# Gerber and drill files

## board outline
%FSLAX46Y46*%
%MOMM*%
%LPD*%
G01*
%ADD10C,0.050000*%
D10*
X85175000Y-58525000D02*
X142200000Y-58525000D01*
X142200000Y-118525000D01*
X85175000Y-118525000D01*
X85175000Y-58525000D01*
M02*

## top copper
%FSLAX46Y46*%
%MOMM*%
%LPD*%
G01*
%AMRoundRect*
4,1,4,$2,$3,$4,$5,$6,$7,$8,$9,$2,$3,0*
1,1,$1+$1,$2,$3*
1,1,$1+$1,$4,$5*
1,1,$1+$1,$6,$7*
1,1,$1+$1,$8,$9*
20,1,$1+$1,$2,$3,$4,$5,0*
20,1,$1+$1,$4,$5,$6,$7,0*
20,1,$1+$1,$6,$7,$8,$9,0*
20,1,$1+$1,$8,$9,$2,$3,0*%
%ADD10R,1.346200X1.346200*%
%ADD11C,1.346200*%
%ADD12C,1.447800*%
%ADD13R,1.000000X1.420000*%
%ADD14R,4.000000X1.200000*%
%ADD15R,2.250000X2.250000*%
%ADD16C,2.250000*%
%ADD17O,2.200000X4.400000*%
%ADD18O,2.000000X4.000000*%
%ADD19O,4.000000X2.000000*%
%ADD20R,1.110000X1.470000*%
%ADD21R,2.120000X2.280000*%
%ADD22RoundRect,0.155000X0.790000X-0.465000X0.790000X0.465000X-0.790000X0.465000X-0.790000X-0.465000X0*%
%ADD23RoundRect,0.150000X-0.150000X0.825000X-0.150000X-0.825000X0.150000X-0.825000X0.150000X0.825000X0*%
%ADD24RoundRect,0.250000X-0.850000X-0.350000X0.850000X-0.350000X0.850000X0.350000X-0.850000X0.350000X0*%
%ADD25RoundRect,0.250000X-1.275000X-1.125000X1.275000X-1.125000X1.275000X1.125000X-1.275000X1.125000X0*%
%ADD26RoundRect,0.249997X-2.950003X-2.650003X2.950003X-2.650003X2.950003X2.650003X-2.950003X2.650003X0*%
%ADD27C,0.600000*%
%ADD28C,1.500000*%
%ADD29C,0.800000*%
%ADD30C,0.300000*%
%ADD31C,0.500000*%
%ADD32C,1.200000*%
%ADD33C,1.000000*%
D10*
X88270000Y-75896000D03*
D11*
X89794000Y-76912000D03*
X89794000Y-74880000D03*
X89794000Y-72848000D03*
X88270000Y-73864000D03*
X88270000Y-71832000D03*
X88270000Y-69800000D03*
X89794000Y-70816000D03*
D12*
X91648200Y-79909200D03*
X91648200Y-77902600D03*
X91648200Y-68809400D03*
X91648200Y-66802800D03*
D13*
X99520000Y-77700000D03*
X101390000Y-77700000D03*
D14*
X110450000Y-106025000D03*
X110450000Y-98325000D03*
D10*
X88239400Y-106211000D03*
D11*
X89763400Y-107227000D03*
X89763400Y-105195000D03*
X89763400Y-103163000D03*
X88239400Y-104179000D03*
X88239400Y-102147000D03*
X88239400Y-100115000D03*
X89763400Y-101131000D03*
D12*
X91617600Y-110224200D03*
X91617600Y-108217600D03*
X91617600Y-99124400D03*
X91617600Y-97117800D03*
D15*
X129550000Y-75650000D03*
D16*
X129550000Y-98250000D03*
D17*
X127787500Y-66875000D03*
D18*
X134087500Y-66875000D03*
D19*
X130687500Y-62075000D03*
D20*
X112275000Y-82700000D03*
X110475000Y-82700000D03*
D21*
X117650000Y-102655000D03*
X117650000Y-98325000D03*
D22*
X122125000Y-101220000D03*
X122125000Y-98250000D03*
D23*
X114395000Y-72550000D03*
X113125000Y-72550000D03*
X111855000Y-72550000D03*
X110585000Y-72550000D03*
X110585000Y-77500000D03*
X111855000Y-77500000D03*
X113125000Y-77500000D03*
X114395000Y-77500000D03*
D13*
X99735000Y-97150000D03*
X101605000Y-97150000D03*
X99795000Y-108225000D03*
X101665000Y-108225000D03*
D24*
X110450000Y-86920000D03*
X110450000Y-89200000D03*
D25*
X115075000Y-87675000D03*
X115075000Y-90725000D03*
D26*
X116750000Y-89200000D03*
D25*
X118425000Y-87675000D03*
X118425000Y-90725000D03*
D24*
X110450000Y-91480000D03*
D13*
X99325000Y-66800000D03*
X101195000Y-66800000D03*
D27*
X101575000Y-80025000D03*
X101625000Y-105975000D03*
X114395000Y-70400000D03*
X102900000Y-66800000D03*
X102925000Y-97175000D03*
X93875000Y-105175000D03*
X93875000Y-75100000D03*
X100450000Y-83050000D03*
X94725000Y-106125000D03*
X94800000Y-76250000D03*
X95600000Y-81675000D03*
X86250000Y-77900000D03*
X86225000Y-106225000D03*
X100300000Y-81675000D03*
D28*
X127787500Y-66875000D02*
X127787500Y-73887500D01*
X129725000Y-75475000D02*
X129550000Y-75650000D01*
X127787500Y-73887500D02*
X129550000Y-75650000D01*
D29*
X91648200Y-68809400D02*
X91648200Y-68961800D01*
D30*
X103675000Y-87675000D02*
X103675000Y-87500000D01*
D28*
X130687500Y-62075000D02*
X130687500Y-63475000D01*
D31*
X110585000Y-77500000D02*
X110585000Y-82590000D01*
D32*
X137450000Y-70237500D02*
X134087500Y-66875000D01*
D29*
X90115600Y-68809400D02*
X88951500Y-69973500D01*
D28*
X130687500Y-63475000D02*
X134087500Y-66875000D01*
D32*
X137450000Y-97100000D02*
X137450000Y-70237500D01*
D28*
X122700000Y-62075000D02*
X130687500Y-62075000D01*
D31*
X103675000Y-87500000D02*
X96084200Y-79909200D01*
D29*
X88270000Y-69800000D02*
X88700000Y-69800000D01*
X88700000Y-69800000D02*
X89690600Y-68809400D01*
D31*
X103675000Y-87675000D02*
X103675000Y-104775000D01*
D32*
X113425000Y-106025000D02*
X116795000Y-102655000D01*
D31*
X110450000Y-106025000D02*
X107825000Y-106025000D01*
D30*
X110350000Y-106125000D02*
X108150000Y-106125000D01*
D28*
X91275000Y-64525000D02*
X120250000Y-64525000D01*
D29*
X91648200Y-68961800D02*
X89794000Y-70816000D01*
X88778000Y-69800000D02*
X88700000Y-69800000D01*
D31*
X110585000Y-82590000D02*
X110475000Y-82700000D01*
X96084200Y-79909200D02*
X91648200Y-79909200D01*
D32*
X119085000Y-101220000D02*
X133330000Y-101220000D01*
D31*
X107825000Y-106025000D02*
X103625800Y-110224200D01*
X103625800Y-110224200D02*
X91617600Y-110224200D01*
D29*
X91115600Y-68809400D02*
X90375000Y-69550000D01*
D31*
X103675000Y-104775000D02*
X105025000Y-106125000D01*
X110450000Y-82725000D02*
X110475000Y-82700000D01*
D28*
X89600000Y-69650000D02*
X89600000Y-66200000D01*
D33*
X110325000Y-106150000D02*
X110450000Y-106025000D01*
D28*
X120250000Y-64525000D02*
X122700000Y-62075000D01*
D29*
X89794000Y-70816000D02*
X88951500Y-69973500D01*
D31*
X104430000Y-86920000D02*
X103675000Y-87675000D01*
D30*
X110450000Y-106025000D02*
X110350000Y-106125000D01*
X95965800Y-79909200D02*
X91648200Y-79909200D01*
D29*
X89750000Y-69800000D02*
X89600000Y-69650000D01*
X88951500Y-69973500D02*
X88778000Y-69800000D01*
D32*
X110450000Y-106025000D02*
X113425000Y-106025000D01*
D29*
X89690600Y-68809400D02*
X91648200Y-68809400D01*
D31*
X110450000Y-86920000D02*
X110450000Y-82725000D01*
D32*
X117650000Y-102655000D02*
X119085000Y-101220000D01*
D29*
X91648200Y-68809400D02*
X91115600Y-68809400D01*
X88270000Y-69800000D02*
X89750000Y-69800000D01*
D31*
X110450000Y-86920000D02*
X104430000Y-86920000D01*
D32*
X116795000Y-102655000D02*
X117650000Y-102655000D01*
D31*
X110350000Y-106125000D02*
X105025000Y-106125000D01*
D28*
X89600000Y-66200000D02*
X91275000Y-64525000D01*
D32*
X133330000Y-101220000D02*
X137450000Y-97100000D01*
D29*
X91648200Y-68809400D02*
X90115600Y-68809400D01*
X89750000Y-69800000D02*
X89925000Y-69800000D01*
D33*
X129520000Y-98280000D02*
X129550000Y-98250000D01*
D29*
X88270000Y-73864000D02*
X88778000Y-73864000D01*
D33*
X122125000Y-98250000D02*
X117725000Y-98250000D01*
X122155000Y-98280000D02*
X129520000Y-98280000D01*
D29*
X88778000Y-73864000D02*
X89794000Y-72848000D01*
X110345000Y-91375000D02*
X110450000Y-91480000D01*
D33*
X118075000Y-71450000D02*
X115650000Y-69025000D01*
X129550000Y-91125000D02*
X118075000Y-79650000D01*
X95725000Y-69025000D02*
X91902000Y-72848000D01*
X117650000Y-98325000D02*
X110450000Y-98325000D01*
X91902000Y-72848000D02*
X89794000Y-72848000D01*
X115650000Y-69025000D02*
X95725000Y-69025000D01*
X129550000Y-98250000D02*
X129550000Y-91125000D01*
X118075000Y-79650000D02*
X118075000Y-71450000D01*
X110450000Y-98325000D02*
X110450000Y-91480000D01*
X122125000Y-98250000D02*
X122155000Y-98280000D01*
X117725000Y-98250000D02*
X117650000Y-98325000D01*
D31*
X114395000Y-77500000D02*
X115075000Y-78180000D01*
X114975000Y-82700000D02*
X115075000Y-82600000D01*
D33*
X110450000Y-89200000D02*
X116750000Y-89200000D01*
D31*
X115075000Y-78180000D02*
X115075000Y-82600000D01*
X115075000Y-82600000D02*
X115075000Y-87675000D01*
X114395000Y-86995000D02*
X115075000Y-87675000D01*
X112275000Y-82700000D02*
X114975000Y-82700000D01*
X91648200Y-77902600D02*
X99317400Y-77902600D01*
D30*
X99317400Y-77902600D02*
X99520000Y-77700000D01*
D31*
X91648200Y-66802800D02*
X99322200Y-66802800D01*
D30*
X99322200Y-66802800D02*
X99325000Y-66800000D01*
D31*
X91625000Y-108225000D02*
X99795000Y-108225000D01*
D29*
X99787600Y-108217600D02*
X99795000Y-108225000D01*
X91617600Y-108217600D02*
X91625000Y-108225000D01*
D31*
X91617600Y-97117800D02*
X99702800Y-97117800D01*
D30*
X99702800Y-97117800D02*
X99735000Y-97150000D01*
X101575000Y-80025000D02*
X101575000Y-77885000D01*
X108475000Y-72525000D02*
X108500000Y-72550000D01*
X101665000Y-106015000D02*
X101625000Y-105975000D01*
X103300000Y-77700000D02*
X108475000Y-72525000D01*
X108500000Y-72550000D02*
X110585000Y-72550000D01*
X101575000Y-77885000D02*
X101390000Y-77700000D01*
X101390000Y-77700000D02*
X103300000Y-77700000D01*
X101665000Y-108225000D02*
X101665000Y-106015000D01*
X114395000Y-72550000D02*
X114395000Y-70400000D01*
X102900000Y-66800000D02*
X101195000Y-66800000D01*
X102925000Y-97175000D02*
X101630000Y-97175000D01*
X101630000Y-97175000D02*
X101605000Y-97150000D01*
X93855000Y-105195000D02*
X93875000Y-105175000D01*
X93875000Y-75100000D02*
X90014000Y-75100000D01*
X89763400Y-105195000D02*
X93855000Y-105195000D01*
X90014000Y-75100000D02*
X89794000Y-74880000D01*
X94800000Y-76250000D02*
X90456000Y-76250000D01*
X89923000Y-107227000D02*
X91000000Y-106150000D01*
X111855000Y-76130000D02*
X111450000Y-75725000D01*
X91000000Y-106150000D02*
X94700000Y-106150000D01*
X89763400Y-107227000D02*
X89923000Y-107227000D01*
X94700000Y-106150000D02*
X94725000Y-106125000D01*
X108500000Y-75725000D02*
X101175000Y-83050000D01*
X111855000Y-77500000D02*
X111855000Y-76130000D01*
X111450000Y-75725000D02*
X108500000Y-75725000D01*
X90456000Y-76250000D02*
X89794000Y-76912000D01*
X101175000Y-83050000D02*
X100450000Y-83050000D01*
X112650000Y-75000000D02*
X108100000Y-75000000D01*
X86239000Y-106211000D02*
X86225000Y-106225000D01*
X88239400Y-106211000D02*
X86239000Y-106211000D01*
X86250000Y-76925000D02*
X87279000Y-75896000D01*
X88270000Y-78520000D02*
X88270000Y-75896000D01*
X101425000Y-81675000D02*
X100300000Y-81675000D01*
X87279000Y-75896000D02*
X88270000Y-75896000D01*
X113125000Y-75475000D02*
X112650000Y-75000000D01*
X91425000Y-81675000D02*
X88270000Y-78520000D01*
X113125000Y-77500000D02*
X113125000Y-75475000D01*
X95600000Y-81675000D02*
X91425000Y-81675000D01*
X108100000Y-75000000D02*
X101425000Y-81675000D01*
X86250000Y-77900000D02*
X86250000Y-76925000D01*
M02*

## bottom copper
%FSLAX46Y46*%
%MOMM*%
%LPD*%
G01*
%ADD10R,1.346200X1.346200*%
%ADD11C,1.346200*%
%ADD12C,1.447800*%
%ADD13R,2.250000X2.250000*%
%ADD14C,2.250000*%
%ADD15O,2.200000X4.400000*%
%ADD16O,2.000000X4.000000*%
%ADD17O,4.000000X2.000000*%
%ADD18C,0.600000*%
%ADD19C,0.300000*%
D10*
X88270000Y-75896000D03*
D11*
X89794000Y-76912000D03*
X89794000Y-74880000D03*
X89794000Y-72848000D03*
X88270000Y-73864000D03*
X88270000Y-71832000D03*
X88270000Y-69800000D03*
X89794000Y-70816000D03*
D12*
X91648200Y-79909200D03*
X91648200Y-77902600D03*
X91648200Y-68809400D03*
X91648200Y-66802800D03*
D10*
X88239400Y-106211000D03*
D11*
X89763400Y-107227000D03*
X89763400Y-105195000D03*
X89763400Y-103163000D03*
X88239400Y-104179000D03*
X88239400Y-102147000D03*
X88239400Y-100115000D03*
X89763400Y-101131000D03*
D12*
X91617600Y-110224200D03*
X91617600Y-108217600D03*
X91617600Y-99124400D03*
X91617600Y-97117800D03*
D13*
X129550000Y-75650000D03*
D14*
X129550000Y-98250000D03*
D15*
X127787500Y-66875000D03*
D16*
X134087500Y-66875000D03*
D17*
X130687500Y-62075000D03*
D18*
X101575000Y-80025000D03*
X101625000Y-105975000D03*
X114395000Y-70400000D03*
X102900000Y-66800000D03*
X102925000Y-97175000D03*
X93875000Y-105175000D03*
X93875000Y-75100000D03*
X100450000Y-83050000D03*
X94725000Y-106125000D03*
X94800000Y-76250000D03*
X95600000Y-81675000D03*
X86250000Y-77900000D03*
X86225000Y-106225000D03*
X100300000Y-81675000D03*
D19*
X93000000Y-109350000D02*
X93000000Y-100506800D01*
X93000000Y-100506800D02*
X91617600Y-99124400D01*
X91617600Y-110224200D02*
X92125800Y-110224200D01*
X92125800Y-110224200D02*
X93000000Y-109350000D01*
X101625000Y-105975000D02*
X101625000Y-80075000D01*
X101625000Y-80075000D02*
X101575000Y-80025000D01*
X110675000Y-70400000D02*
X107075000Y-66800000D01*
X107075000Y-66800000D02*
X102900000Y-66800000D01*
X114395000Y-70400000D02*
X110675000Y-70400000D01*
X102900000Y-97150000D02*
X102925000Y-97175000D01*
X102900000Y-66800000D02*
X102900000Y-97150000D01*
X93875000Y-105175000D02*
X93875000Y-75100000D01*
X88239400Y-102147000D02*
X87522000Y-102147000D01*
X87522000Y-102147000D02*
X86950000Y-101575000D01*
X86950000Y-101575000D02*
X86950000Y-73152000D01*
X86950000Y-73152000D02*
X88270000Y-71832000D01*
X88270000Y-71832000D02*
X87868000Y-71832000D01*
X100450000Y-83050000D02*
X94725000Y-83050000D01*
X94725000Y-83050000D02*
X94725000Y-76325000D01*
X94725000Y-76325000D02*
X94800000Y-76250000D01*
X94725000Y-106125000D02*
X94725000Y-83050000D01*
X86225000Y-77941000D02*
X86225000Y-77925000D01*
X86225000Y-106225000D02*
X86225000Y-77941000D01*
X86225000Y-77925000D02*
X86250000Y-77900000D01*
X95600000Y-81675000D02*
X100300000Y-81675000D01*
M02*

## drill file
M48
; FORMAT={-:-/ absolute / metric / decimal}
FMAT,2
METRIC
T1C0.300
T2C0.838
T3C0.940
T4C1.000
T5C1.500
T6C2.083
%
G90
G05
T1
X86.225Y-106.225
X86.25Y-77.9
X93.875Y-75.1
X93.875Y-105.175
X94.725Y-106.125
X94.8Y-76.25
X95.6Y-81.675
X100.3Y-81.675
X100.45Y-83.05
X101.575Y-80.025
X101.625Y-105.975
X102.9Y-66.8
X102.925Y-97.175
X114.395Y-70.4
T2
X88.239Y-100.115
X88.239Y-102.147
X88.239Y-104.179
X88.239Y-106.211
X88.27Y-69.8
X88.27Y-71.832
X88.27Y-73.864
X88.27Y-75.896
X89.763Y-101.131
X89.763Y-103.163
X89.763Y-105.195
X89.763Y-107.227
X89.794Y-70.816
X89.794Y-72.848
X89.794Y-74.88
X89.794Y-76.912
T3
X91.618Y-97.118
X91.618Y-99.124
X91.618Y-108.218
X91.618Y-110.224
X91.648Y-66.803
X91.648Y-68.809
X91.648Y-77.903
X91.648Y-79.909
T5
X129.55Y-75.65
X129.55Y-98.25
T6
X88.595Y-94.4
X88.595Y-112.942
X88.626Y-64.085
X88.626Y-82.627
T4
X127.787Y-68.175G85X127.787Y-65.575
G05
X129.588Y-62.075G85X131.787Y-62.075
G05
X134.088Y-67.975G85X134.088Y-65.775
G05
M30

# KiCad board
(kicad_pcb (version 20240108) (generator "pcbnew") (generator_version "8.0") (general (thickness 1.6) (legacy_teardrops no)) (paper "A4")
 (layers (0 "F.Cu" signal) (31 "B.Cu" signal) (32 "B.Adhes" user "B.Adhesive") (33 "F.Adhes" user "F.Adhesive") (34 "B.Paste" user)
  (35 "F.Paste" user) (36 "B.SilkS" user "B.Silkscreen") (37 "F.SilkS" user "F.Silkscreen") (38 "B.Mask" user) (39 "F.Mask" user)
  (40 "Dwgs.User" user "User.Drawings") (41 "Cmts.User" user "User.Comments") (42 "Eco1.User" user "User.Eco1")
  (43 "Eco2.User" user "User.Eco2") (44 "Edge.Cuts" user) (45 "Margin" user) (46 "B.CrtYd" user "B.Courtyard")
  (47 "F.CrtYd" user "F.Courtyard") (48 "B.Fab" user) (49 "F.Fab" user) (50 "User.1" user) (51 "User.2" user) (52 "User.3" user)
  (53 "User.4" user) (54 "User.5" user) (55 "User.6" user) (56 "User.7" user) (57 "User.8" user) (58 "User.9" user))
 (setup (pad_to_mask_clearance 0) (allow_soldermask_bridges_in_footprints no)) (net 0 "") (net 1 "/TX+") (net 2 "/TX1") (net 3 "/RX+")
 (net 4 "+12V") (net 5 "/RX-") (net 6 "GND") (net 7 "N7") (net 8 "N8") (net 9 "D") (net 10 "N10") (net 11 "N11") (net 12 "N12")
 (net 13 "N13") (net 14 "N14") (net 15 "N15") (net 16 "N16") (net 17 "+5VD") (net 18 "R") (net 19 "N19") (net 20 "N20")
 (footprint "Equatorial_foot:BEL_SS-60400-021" (layer "F.Cu") (at 88.6256 73.356 -90)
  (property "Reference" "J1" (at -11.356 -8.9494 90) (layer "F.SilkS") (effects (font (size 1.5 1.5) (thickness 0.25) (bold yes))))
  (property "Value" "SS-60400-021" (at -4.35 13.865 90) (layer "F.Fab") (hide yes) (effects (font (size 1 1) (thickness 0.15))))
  (pad "" np_thru_hole circle (at -9.271 0 270) (size 2.0828 2.0828) (drill 2.0828) (layers "*.Cu" "*.Mask"))
  (pad "" np_thru_hole circle (at 9.271 0 270) (size 2.0828 2.0828) (drill 2.0828) (layers "*.Cu" "*.Mask"))
  (pad "1" thru_hole rect (at 2.54 0.3556 270) (size 1.3462 1.3462) (drill 0.8382) (layers "*.Cu" "*.Mask") (remove_unused_layers no)
   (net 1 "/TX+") (solder_mask_margin 0.102))
  (pad "2" thru_hole circle (at 3.556 -1.1684 270) (size 1.3462 1.3462) (drill 0.8382) (layers "*.Cu" "*.Mask") (remove_unused_layers no)
   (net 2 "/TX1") (solder_mask_margin 0.102))
  (pad "3" thru_hole circle (at 1.524 -1.1684 270) (size 1.3462 1.3462) (drill 0.8382) (layers "*.Cu" "*.Mask") (remove_unused_layers no)
   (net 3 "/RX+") (solder_mask_margin 0.102))
  (pad "4" thru_hole circle (at -0.508 -1.1684 270) (size 1.3462 1.3462) (drill 0.8382) (layers "*.Cu" "*.Mask") (remove_unused_layers no)
   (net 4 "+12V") (solder_mask_margin 0.102))
  (pad "5" thru_hole circle (at 0.508 0.3556 270) (size 1.3462 1.3462) (drill 0.8382) (layers "*.Cu" "*.Mask") (remove_unused_layers no)
   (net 4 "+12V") (solder_mask_margin 0.102))
  (pad "6" thru_hole circle (at -1.524 0.3556 270) (size 1.3462 1.3462) (drill 0.8382) (layers "*.Cu" "*.Mask") (remove_unused_layers no)
   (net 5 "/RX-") (solder_mask_margin 0.102))
  (pad "7" thru_hole circle (at -3.556 0.3556 270) (size 1.3462 1.3462) (drill 0.8382) (layers "*.Cu" "*.Mask") (remove_unused_layers no)
   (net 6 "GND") (solder_mask_margin 0.102))
  (pad "8" thru_hole circle (at -2.54 -1.1684 270) (size 1.3462 1.3462) (drill 0.8382) (layers "*.Cu" "*.Mask") (remove_unused_layers no)
   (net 6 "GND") (solder_mask_margin 0.102))
  (pad "9" thru_hole circle (at 6.5532 -3.0226 270) (size 1.4478 1.4478) (drill 0.9398) (layers "*.Cu" "*.Mask") (remove_unused_layers no)
   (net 6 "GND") (solder_mask_margin 0.102))
  (pad "10" thru_hole circle (at 4.5466 -3.0226 270) (size 1.4478 1.4478) (drill 0.9398) (layers "*.Cu" "*.Mask") (remove_unused_layers no)
   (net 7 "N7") (solder_mask_margin 0.102))
  (pad "11" thru_hole circle (at -4.5466 -3.0226 270) (size 1.4478 1.4478) (drill 0.9398) (layers "*.Cu" "*.Mask") (remove_unused_layers no)
   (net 6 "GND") (solder_mask_margin 0.102))
  (pad "12" thru_hole circle (at -6.5532 -3.0226 270) (size 1.4478 1.4478) (drill 0.9398) (layers "*.Cu" "*.Mask") (remove_unused_layers no)
   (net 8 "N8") (solder_mask_margin 0.102)))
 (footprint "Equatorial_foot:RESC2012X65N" (layer "F.Cu") (at 100.455 77.7)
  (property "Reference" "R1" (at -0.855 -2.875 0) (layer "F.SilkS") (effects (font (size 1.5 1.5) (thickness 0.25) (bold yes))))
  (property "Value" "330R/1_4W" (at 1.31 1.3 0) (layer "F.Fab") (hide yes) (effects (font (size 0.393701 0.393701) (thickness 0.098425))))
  (pad "1" smd rect (at -0.935 0) (size 1 1.42) (layers "F.Cu" "F.Paste" "F.Mask") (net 7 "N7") (solder_mask_margin 0.102))
  (pad "2" smd rect (at 0.935 0) (size 1 1.42) (layers "F.Cu" "F.Paste" "F.Mask") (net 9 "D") (solder_mask_margin 0.102)))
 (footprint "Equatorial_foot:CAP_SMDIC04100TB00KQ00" (layer "F.Cu") (at 110.45 102.175 90)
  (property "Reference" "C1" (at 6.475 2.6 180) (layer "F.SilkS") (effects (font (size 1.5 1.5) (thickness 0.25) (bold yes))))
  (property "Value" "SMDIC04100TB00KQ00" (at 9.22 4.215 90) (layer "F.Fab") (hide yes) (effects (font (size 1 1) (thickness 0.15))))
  (pad "1" smd rect (at -3.85 0 90) (size 1.2 4) (layers "F.Cu" "F.Paste" "F.Mask") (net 6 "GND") (solder_mask_margin 0.102))
  (pad "2" smd rect (at 3.85 0 90) (size 1.2 4) (layers "F.Cu" "F.Paste" "F.Mask") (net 4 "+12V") (solder_mask_margin 0.102)))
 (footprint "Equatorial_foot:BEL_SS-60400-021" (layer "F.Cu") (at 88.595 103.671 -90)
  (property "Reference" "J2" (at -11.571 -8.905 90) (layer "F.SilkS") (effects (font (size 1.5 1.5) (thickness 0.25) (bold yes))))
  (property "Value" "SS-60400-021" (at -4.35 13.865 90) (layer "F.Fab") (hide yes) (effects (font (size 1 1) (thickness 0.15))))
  (pad "" np_thru_hole circle (at -9.271 0 270) (size 2.0828 2.0828) (drill 2.0828) (layers "*.Cu" "*.Mask"))
  (pad "" np_thru_hole circle (at 9.271 0 270) (size 2.0828 2.0828) (drill 2.0828) (layers "*.Cu" "*.Mask"))
  (pad "1" thru_hole rect (at 2.54 0.3556 270) (size 1.3462 1.3462) (drill 0.8382) (layers "*.Cu" "*.Mask") (remove_unused_layers no)
   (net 1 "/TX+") (solder_mask_margin 0.102))
  (pad "2" thru_hole circle (at 3.556 -1.1684 270) (size 1.3462 1.3462) (drill 0.8382) (layers "*.Cu" "*.Mask") (remove_unused_layers no)
   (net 2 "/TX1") (solder_mask_margin 0.102))
  (pad "3" thru_hole circle (at 1.524 -1.1684 270) (size 1.3462 1.3462) (drill 0.8382) (layers "*.Cu" "*.Mask") (remove_unused_layers no)
   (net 3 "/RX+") (solder_mask_margin 0.102))
  (pad "4" thru_hole circle (at -0.508 -1.1684 270) (size 1.3462 1.3462) (drill 0.8382) (layers "*.Cu" "*.Mask") (remove_unused_layers no)
   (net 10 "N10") (solder_mask_margin 0.102))
  (pad "5" thru_hole circle (at 0.508 0.3556 270) (size 1.3462 1.3462) (drill 0.8382) (layers "*.Cu" "*.Mask") (remove_unused_layers no)
   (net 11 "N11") (solder_mask_margin 0.102))
  (pad "6" thru_hole circle (at -1.524 0.3556 270) (size 1.3462 1.3462) (drill 0.8382) (layers "*.Cu" "*.Mask") (remove_unused_layers no)
   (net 5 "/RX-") (solder_mask_margin 0.102))
  (pad "7" thru_hole circle (at -3.556 0.3556 270) (size 1.3462 1.3462) (drill 0.8382) (layers "*.Cu" "*.Mask") (remove_unused_layers no)
   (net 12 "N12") (solder_mask_margin 0.102))
  (pad "8" thru_hole circle (at -2.54 -1.1684 270) (size 1.3462 1.3462) (drill 0.8382) (layers "*.Cu" "*.Mask") (remove_unused_layers no)
   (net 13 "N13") (solder_mask_margin 0.102))
  (pad "9" thru_hole circle (at 6.5532 -3.0226 270) (size 1.4478 1.4478) (drill 0.9398) (layers "*.Cu" "*.Mask") (remove_unused_layers no)
   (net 6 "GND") (solder_mask_margin 0.102))
  (pad "10" thru_hole circle (at 4.5466 -3.0226 270) (size 1.4478 1.4478) (drill 0.9398) (layers "*.Cu" "*.Mask") (remove_unused_layers no)
   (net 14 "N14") (solder_mask_margin 0.102))
  (pad "11" thru_hole circle (at -4.5466 -3.0226 270) (size 1.4478 1.4478) (drill 0.9398) (layers "*.Cu" "*.Mask") (remove_unused_layers no)
   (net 6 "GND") (solder_mask_margin 0.102))
  (pad "12" thru_hole circle (at -6.5532 -3.0226 270) (size 1.4478 1.4478) (drill 0.9398) (layers "*.Cu" "*.Mask") (remove_unused_layers no)
   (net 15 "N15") (solder_mask_margin 0.102)))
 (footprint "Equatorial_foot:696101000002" (layer "F.Cu") (at 129.55 75.65 -90)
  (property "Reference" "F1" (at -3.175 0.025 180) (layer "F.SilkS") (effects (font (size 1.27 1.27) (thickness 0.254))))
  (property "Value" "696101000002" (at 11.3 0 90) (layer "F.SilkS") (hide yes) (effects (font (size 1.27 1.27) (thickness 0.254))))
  (pad "1" thru_hole rect (at 0 0 270) (size 2.25 2.25) (drill 1.5) (layers "*.Cu" "*.Mask") (remove_unused_layers no) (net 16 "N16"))
  (pad "2" thru_hole circle (at 22.6 0 270) (size 2.25 2.25) (drill 1.5) (layers "*.Cu" "*.Mask") (remove_unused_layers no) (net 4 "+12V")))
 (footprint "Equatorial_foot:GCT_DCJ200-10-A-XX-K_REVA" (layer "F.Cu") (at 134.3375 66.875 90)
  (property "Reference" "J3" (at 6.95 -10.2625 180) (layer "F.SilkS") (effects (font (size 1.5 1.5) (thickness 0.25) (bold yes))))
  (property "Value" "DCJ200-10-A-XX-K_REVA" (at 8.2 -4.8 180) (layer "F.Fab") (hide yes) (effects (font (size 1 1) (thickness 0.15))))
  (pad "1" thru_hole oval (at 0 -6.55 90) (size 4.4 2.2) (drill oval 3.6 1) (layers "*.Cu" "*.Mask") (remove_unused_layers no)
   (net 16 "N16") (solder_mask_margin 0.102))
  (pad "2" thru_hole oval (at 0 -0.25 90) (size 4 2) (drill oval 3.2 1) (layers "*.Cu" "*.Mask") (remove_unused_layers no) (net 6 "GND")
   (solder_mask_margin 0.102))
  (pad "3" thru_hole oval (at 4.8 -3.65 90) (size 2 4) (drill oval 1 3.2) (layers "*.Cu" "*.Mask") (remove_unused_layers no) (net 6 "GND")
   (solder_mask_margin 0.102)))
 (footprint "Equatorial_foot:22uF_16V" (layer "F.Cu") (at 111.375 82.7 180)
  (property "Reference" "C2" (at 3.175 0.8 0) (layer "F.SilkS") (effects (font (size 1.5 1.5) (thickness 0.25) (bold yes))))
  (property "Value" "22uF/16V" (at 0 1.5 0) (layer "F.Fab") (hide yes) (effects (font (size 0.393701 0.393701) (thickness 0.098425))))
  (pad "1" smd rect (at -0.9 0 180) (size 1.11 1.47) (layers "F.Cu" "F.Paste" "F.Mask") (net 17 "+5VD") (solder_mask_margin 0.102))
  (pad "2" smd rect (at 0.9 0 180) (size 1.11 1.47) (layers "F.Cu" "F.Paste" "F.Mask") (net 6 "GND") (solder_mask_margin 0.102)))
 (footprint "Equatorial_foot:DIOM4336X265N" (layer "F.Cu") (at 117.65 100.49 -90)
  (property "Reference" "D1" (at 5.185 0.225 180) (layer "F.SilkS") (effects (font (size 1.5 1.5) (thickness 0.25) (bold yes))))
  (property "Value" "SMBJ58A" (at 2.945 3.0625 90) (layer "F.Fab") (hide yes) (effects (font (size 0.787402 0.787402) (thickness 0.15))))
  (pad "A" smd rect (at 2.165 0 270) (size 2.28 2.12) (layers "F.Cu" "F.Paste" "F.Mask") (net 6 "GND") (solder_mask_margin 0.102))
  (pad "C" smd rect (at -2.165 0 270) (size 2.28 2.12) (layers "F.Cu" "F.Paste" "F.Mask") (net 4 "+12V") (solder_mask_margin 0.102)))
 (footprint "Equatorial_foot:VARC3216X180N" (layer "F.Cu") (at 122.125 99.735 90)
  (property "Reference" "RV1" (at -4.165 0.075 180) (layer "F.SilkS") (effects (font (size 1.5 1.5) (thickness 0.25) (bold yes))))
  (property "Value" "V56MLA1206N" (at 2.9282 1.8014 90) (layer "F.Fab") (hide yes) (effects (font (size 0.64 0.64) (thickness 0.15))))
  (pad "1" smd roundrect (at -1.485 0 90) (size 1.24 1.89) (layers "F.Cu" "F.Paste" "F.Mask") (roundrect_rratio 0.125) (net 6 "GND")
   (solder_mask_margin 0.102))
  (pad "2" smd roundrect (at 1.485 0 90) (size 1.24 1.89) (layers "F.Cu" "F.Paste" "F.Mask") (roundrect_rratio 0.125) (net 4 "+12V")
   (solder_mask_margin 0.102)))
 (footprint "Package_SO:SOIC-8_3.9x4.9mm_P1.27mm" (layer "F.Cu") (at 112.49 75.025 -90)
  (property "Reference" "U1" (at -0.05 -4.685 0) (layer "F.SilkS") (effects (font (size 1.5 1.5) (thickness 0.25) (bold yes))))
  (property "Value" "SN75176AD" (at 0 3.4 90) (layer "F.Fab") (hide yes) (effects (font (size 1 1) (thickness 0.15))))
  (pad "1" smd roundrect (at -2.475 -1.905 270) (size 1.95 0.6) (layers "F.Cu" "F.Paste" "F.Mask") (roundrect_rratio 0.25) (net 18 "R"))
  (pad "2" smd roundrect (at -2.475 -0.635 270) (size 1.95 0.6) (layers "F.Cu" "F.Paste" "F.Mask") (roundrect_rratio 0.25) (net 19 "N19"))
  (pad "3" smd roundrect (at -2.475 0.635 270) (size 1.95 0.6) (layers "F.Cu" "F.Paste" "F.Mask") (roundrect_rratio 0.25) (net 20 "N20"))
  (pad "4" smd roundrect (at -2.475 1.905 270) (size 1.95 0.6) (layers "F.Cu" "F.Paste" "F.Mask") (roundrect_rratio 0.25) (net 9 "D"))
  (pad "5" smd roundrect (at 2.475 1.905 270) (size 1.95 0.6) (layers "F.Cu" "F.Paste" "F.Mask") (roundrect_rratio 0.25) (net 6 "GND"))
  (pad "6" smd roundrect (at 2.475 0.635 270) (size 1.95 0.6) (layers "F.Cu" "F.Paste" "F.Mask") (roundrect_rratio 0.25) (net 2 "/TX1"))
  (pad "7" smd roundrect (at 2.475 -0.635 270) (size 1.95 0.6) (layers "F.Cu" "F.Paste" "F.Mask") (roundrect_rratio 0.25) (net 1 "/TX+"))
  (pad "8" smd roundrect (at 2.475 -1.905 270) (size 1.95 0.6) (layers "F.Cu" "F.Paste" "F.Mask") (roundrect_rratio 0.25) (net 17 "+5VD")))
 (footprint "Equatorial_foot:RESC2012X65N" (layer "F.Cu") (at 100.67 97.15)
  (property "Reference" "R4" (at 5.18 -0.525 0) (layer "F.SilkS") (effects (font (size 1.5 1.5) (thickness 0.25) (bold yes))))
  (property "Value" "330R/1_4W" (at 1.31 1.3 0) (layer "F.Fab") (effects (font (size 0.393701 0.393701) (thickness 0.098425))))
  (pad "1" smd rect (at -0.935 0) (size 1 1.42) (layers "F.Cu" "F.Paste" "F.Mask") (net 15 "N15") (solder_mask_margin 0.102))
  (pad "2" smd rect (at 0.935 0) (size 1 1.42) (layers "F.Cu" "F.Paste" "F.Mask") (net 18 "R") (solder_mask_margin 0.102)))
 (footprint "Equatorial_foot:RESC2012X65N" (layer "F.Cu") (at 100.73 108.225)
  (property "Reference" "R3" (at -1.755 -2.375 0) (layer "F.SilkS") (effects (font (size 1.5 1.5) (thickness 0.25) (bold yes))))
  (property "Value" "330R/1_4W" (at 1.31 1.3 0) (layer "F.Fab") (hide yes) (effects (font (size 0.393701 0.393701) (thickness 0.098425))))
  (pad "1" smd rect (at -0.935 0) (size 1 1.42) (layers "F.Cu" "F.Paste" "F.Mask") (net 14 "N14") (solder_mask_margin 0.102))
  (pad "2" smd rect (at 0.935 0) (size 1 1.42) (layers "F.Cu" "F.Paste" "F.Mask") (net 9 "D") (solder_mask_margin 0.102)))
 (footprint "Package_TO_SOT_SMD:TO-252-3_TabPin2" (layer "F.Cu") (at 115.49 89.2)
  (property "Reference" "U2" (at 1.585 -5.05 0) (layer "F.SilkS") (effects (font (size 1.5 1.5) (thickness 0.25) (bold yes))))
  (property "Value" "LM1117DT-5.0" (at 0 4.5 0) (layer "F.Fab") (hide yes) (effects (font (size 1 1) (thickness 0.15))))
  (pad "1" smd roundrect (at -5.04 -2.28) (size 2.2 1.2) (layers "F.Cu" "F.Paste" "F.Mask") (roundrect_rratio 0.208333) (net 6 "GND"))
  (pad "2" smd roundrect (at -5.04 0) (size 2.2 1.2) (layers "F.Cu" "F.Paste" "F.Mask") (roundrect_rratio 0.208333) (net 17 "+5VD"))
  (pad "2" smd roundrect (at -0.415 -1.525) (size 3.05 2.75) (layers "F.Cu" "F.Paste") (roundrect_rratio 0.090909) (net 17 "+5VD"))
  (pad "2" smd roundrect (at -0.415 1.525) (size 3.05 2.75) (layers "F.Cu" "F.Paste") (roundrect_rratio 0.090909) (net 17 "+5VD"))
  (pad "2" smd roundrect (at 1.26 0) (size 6.4 5.8) (layers "F.Cu" "F.Mask") (roundrect_rratio 0.043103) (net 17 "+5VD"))
  (pad "2" smd roundrect (at 2.935 -1.525) (size 3.05 2.75) (layers "F.Cu" "F.Paste") (roundrect_rratio 0.090909) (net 17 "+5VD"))
  (pad "2" smd roundrect (at 2.935 1.525) (size 3.05 2.75) (layers "F.Cu" "F.Paste") (roundrect_rratio 0.090909) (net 17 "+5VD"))
  (pad "3" smd roundrect (at -5.04 2.28) (size 2.2 1.2) (layers "F.Cu" "F.Paste" "F.Mask") (roundrect_rratio 0.208333) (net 4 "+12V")))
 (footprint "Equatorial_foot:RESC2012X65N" (layer "F.Cu") (at 100.26 66.8)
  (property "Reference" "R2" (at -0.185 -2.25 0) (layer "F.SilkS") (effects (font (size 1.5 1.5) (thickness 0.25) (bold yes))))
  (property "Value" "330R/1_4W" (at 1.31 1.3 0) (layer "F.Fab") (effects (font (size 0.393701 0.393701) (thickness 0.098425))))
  (pad "1" smd rect (at -0.935 0) (size 1 1.42) (layers "F.Cu" "F.Paste" "F.Mask") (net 8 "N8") (solder_mask_margin 0.102))
  (pad "2" smd rect (at 0.935 0) (size 1 1.42) (layers "F.Cu" "F.Paste" "F.Mask") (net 18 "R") (solder_mask_margin 0.102)))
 (gr_rect (start 85.175 58.525) (end 142.2 118.525) (stroke (width 0.05) (type default)) (fill none) (layer "Edge.Cuts"))
 (segment (start 127.7875 66.875) (end 127.7875 73.8875) (width 1.5) (layer "F.Cu") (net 16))
 (segment (start 129.725 75.475) (end 129.55 75.65) (width 1.5) (layer "F.Cu") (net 16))
 (segment (start 127.7875 73.8875) (end 129.55 75.65) (width 1.5) (layer "F.Cu") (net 16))
 (segment (start 91.6482 68.8094) (end 91.6482 68.9618) (width 0.8) (layer "F.Cu") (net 6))
 (segment (start 103.675 87.675) (end 103.675 87.5) (width 0.3) (layer "F.Cu") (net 6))
 (segment (start 130.6875 62.075) (end 130.6875 63.475) (width 1.5) (layer "F.Cu") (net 6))
 (segment (start 110.585 77.5) (end 110.585 82.59) (width 0.5) (layer "F.Cu") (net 6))
 (segment (start 137.45 70.2375) (end 134.0875 66.875) (width 1.2) (layer "F.Cu") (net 6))
 (segment (start 90.1156 68.8094) (end 88.9515 69.9735) (width 0.8) (layer "F.Cu") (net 6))
 (segment (start 130.6875 63.475) (end 134.0875 66.875) (width 1.5) (layer "F.Cu") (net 6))
 (segment (start 137.45 97.1) (end 137.45 70.2375) (width 1.2) (layer "F.Cu") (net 6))
 (segment (start 122.7 62.075) (end 130.6875 62.075) (width 1.5) (layer "F.Cu") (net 6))
 (segment (start 103.675 87.5) (end 96.0842 79.9092) (width 0.5) (layer "F.Cu") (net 6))
 (segment (start 88.27 69.8) (end 88.7 69.8) (width 0.8) (layer "F.Cu") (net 6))
 (segment (start 88.7 69.8) (end 89.6906 68.8094) (width 0.8) (layer "F.Cu") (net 6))
 (segment (start 103.675 87.675) (end 103.675 104.775) (width 0.5) (layer "F.Cu") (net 6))
 (segment (start 113.425 106.025) (end 116.795 102.655) (width 1.2) (layer "F.Cu") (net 6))
 (segment (start 110.45 106.025) (end 107.825 106.025) (width 0.5) (layer "F.Cu") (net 6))
 (segment (start 110.35 106.125) (end 108.15 106.125) (width 0.3) (layer "F.Cu") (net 6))
 (segment (start 91.275 64.525) (end 120.25 64.525) (width 1.5) (layer "F.Cu") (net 6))
 (segment (start 91.6482 68.9618) (end 89.794 70.816) (width 0.8) (layer "F.Cu") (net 6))
 (segment (start 88.778 69.8) (end 88.7 69.8) (width 0.8) (layer "F.Cu") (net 6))
 (segment (start 110.585 82.59) (end 110.475 82.7) (width 0.5) (layer "F.Cu") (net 6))
 (segment (start 96.0842 79.9092) (end 91.6482 79.9092) (width 0.5) (layer "F.Cu") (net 6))
 (segment (start 119.085 101.22) (end 133.33 101.22) (width 1.2) (layer "F.Cu") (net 6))
 (segment (start 107.825 106.025) (end 103.6258 110.2242) (width 0.5) (layer "F.Cu") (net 6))
 (segment (start 103.6258 110.2242) (end 91.6176 110.2242) (width 0.5) (layer "F.Cu") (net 6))
 (segment (start 91.1156 68.8094) (end 90.375 69.55) (width 0.8) (layer "F.Cu") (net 6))
 (segment (start 103.675 104.775) (end 105.025 106.125) (width 0.5) (layer "F.Cu") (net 6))
 (segment (start 110.45 82.725) (end 110.475 82.7) (width 0.5) (layer "F.Cu") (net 6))
 (segment (start 89.6 69.65) (end 89.6 66.2) (width 1.5) (layer "F.Cu") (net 6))
 (segment (start 110.325 106.15) (end 110.45 106.025) (width 1) (layer "F.Cu") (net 6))
 (segment (start 120.25 64.525) (end 122.7 62.075) (width 1.5) (layer "F.Cu") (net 6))
 (segment (start 89.794 70.816) (end 88.9515 69.9735) (width 0.8) (layer "F.Cu") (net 6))
 (segment (start 104.43 86.92) (end 103.675 87.675) (width 0.5) (layer "F.Cu") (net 6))
 (segment (start 110.45 106.025) (end 110.35 106.125) (width 0.3) (layer "F.Cu") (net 6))
 (segment (start 95.9658 79.9092) (end 91.6482 79.9092) (width 0.3) (layer "F.Cu") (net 6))
 (segment (start 89.75 69.8) (end 89.6 69.65) (width 0.8) (layer "F.Cu") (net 6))
 (segment (start 88.9515 69.9735) (end 88.778 69.8) (width 0.8) (layer "F.Cu") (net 6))
 (segment (start 110.45 106.025) (end 113.425 106.025) (width 1.2) (layer "F.Cu") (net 6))
 (segment (start 89.6906 68.8094) (end 91.6482 68.8094) (width 0.8) (layer "F.Cu") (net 6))
 (segment (start 110.45 86.92) (end 110.45 82.725) (width 0.5) (layer "F.Cu") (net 6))
 (segment (start 117.65 102.655) (end 119.085 101.22) (width 1.2) (layer "F.Cu") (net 6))
 (segment (start 91.6482 68.8094) (end 91.1156 68.8094) (width 0.8) (layer "F.Cu") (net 6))
 (segment (start 88.27 69.8) (end 89.75 69.8) (width 0.8) (layer "F.Cu") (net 6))
 (segment (start 110.45 86.92) (end 104.43 86.92) (width 0.5) (layer "F.Cu") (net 6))
 (segment (start 116.795 102.655) (end 117.65 102.655) (width 1.2) (layer "F.Cu") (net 6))
 (segment (start 110.35 106.125) (end 105.025 106.125) (width 0.5) (layer "F.Cu") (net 6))
 (segment (start 89.6 66.2) (end 91.275 64.525) (width 1.5) (layer "F.Cu") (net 6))
 (segment (start 133.33 101.22) (end 137.45 97.1) (width 1.2) (layer "F.Cu") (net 6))
 (segment (start 91.6482 68.8094) (end 90.1156 68.8094) (width 0.8) (layer "F.Cu") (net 6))
 (segment (start 89.75 69.8) (end 89.925 69.8) (width 0.8) (layer "F.Cu") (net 6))
 (segment (start 93 109.35) (end 93 100.5068) (width 0.3) (layer "B.Cu") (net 6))
 (segment (start 93 100.5068) (end 91.6176 99.1244) (width 0.3) (layer "B.Cu") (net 6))
 (segment (start 91.6176 110.2242) (end 92.1258 110.2242) (width 0.3) (layer "B.Cu") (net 6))
 (segment (start 92.1258 110.2242) (end 93 109.35) (width 0.3) (layer "B.Cu") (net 6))
 (segment (start 129.52 98.28) (end 129.55 98.25) (width 1) (layer "F.Cu") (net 4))
 (segment (start 88.27 73.864) (end 88.778 73.864) (width 0.8) (layer "F.Cu") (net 4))
 (segment (start 122.125 98.25) (end 117.725 98.25) (width 1) (layer "F.Cu") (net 4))
 (segment (start 122.155 98.28) (end 129.52 98.28) (width 1) (layer "F.Cu") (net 4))
 (segment (start 88.778 73.864) (end 89.794 72.848) (width 0.8) (layer "F.Cu") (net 4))
 (segment (start 110.345 91.375) (end 110.45 91.48) (width 0.8) (layer "F.Cu") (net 4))
 (segment (start 118.075 71.45) (end 115.65 69.025) (width 1) (layer "F.Cu") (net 4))
 (segment (start 129.55 91.125) (end 118.075 79.65) (width 1) (layer "F.Cu") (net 4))
 (segment (start 95.725 69.025) (end 91.902 72.848) (width 1) (layer "F.Cu") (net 4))
 (segment (start 117.65 98.325) (end 110.45 98.325) (width 1) (layer "F.Cu") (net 4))
 (segment (start 91.902 72.848) (end 89.794 72.848) (width 1) (layer "F.Cu") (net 4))
 (segment (start 115.65 69.025) (end 95.725 69.025) (width 1) (layer "F.Cu") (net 4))
 (segment (start 129.55 98.25) (end 129.55 91.125) (width 1) (layer "F.Cu") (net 4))
 (segment (start 118.075 79.65) (end 118.075 71.45) (width 1) (layer "F.Cu") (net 4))
 (segment (start 110.45 98.325) (end 110.45 91.48) (width 1) (layer "F.Cu") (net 4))
 (segment (start 122.125 98.25) (end 122.155 98.28) (width 1) (layer "F.Cu") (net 4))
 (segment (start 117.725 98.25) (end 117.65 98.325) (width 1) (layer "F.Cu") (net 4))
 (segment (start 114.395 77.5) (end 115.075 78.18) (width 0.5) (layer "F.Cu") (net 17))
 (segment (start 114.975 82.7) (end 115.075 82.6) (width 0.5) (layer "F.Cu") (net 17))
 (segment (start 110.45 89.2) (end 116.75 89.2) (width 1) (layer "F.Cu") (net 17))
 (segment (start 115.075 78.18) (end 115.075 82.6) (width 0.5) (layer "F.Cu") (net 17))
 (segment (start 115.075 82.6) (end 115.075 87.675) (width 0.5) (layer "F.Cu") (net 17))
 (segment (start 114.395 86.995) (end 115.075 87.675) (width 0.5) (layer "F.Cu") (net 17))
 (segment (start 112.275 82.7) (end 114.975 82.7) (width 0.5) (layer "F.Cu") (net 17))
 (segment (start 91.6482 77.9026) (end 99.3174 77.9026) (width 0.5) (layer "F.Cu") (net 7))
 (segment (start 99.3174 77.9026) (end 99.52 77.7) (width 0.3) (layer "F.Cu") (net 7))
 (segment (start 91.6482 66.8028) (end 99.3222 66.8028) (width 0.5) (layer "F.Cu") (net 8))
 (segment (start 99.3222 66.8028) (end 99.325 66.8) (width 0.3) (layer "F.Cu") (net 8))
 (segment (start 91.625 108.225) (end 99.795 108.225) (width 0.5) (layer "F.Cu") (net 14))
 (segment (start 99.7876 108.2176) (end 99.795 108.225) (width 0.8) (layer "F.Cu") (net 14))
 (segment (start 91.6176 108.2176) (end 91.625 108.225) (width 0.8) (layer "F.Cu") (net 14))
 (segment (start 91.6176 97.1178) (end 99.7028 97.1178) (width 0.5) (layer "F.Cu") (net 15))
 (segment (start 99.7028 97.1178) (end 99.735 97.15) (width 0.3) (layer "F.Cu") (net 15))
 (segment (start 101.575 80.025) (end 101.575 77.885) (width 0.3) (layer "F.Cu") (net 9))
 (segment (start 108.475 72.525) (end 108.5 72.55) (width 0.3) (layer "F.Cu") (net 9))
 (segment (start 101.665 106.015) (end 101.625 105.975) (width 0.3) (layer "F.Cu") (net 9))
 (segment (start 103.3 77.7) (end 108.475 72.525) (width 0.3) (layer "F.Cu") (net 9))
 (segment (start 108.5 72.55) (end 110.585 72.55) (width 0.3) (layer "F.Cu") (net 9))
 (segment (start 101.575 77.885) (end 101.39 77.7) (width 0.3) (layer "F.Cu") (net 9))
 (segment (start 101.39 77.7) (end 103.3 77.7) (width 0.3) (layer "F.Cu") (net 9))
 (segment (start 101.665 108.225) (end 101.665 106.015) (width 0.3) (layer "F.Cu") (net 9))
 (via (at 101.575 80.025) (size 0.6) (drill 0.3) (layers "F.Cu" "B.Cu") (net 9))
 (via (at 101.625 105.975) (size 0.6) (drill 0.3) (layers "F.Cu" "B.Cu") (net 9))
 (segment (start 101.625 105.975) (end 101.625 80.075) (width 0.3) (layer "B.Cu") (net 9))
 (segment (start 101.625 80.075) (end 101.575 80.025) (width 0.3) (layer "B.Cu") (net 9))
 (segment (start 114.395 72.55) (end 114.395 70.4) (width 0.3) (layer "F.Cu") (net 18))
 (segment (start 102.9 66.8) (end 101.195 66.8) (width 0.3) (layer "F.Cu") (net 18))
 (segment (start 102.925 97.175) (end 101.63 97.175) (width 0.3) (layer "F.Cu") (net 18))
 (segment (start 101.63 97.175) (end 101.605 97.15) (width 0.3) (layer "F.Cu") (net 18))
 (via (at 114.395 70.4) (size 0.6) (drill 0.3) (layers "F.Cu" "B.Cu") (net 18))
 (via (at 102.9 66.8) (size 0.6) (drill 0.3) (layers "F.Cu" "B.Cu") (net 18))
 (via (at 102.925 97.175) (size 0.6) (drill 0.3) (layers "F.Cu" "B.Cu") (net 18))
 (segment (start 110.675 70.4) (end 107.075 66.8) (width 0.3) (layer "B.Cu") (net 18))
 (segment (start 107.075 66.8) (end 102.9 66.8) (width 0.3) (layer "B.Cu") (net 18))
 (segment (start 114.395 70.4) (end 110.675 70.4) (width 0.3) (layer "B.Cu") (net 18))
 (segment (start 102.9 97.15) (end 102.925 97.175) (width 0.3) (layer "B.Cu") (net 18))
 (segment (start 102.9 66.8) (end 102.9 97.15) (width 0.3) (layer "B.Cu") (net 18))
 (segment (start 93.855 105.195) (end 93.875 105.175) (width 0.3) (layer "F.Cu") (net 3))
 (segment (start 93.875 75.1) (end 90.014 75.1) (width 0.3) (layer "F.Cu") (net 3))
 (segment (start 89.7634 105.195) (end 93.855 105.195) (width 0.3) (layer "F.Cu") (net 3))
 (segment (start 90.014 75.1) (end 89.794 74.88) (width 0.3) (layer "F.Cu") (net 3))
 (via (at 93.875 105.175) (size 0.6) (drill 0.3) (layers "F.Cu" "B.Cu") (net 3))
 (via (at 93.875 75.1) (size 0.6) (drill 0.3) (layers "F.Cu" "B.Cu") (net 3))
 (segment (start 93.875 105.175) (end 93.875 75.1) (width 0.3) (layer "B.Cu") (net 3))
 (segment (start 88.2394 102.147) (end 87.522 102.147) (width 0.3) (layer "B.Cu") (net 5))
 (segment (start 87.522 102.147) (end 86.95 101.575) (width 0.3) (layer "B.Cu") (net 5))
 (segment (start 86.95 101.575) (end 86.95 73.152) (width 0.3) (layer "B.Cu") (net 5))
 (segment (start 86.95 73.152) (end 88.27 71.832) (width 0.3) (layer "B.Cu") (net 5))
 (segment (start 88.27 71.832) (end 87.868 71.832) (width 0.3) (layer "B.Cu") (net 5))
 (segment (start 94.8 76.25) (end 90.456 76.25) (width 0.3) (layer "F.Cu") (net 2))
 (segment (start 89.923 107.227) (end 91 106.15) (width 0.3) (layer "F.Cu") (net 2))
 (segment (start 111.855 76.13) (end 111.45 75.725) (width 0.3) (layer "F.Cu") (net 2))
 (segment (start 91 106.15) (end 94.7 106.15) (width 0.3) (layer "F.Cu") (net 2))
 (segment (start 89.7634 107.227) (end 89.923 107.227) (width 0.3) (layer "F.Cu") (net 2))
 (segment (start 94.7 106.15) (end 94.725 106.125) (width 0.3) (layer "F.Cu") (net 2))
 (segment (start 108.5 75.725) (end 101.175 83.05) (width 0.3) (layer "F.Cu") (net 2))
 (segment (start 111.855 77.5) (end 111.855 76.13) (width 0.3) (layer "F.Cu") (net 2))
 (segment (start 111.45 75.725) (end 108.5 75.725) (width 0.3) (layer "F.Cu") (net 2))
 (segment (start 90.456 76.25) (end 89.794 76.912) (width 0.3) (layer "F.Cu") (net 2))
 (segment (start 101.175 83.05) (end 100.45 83.05) (width 0.3) (layer "F.Cu") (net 2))
 (via (at 100.45 83.05) (size 0.6) (drill 0.3) (layers "F.Cu" "B.Cu") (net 2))
 (via (at 94.725 106.125) (size 0.6) (drill 0.3) (layers "F.Cu" "B.Cu") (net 2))
 (via (at 94.8 76.25) (size 0.6) (drill 0.3) (layers "F.Cu" "B.Cu") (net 2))
 (segment (start 100.45 83.05) (end 94.725 83.05) (width 0.3) (layer "B.Cu") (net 2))
 (segment (start 94.725 83.05) (end 94.725 76.325) (width 0.3) (layer "B.Cu") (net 2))
 (segment (start 94.725 76.325) (end 94.8 76.25) (width 0.3) (layer "B.Cu") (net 2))
 (segment (start 94.725 106.125) (end 94.725 83.05) (width 0.3) (layer "B.Cu") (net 2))
 (segment (start 112.65 75) (end 108.1 75) (width 0.3) (layer "F.Cu") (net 1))
 (segment (start 86.239 106.211) (end 86.225 106.225) (width 0.3) (layer "F.Cu") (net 1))
 (segment (start 88.2394 106.211) (end 86.239 106.211) (width 0.3) (layer "F.Cu") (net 1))
 (segment (start 86.25 76.925) (end 87.279 75.896) (width 0.3) (layer "F.Cu") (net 1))
 (segment (start 88.27 78.52) (end 88.27 75.896) (width 0.3) (layer "F.Cu") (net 1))
 (segment (start 101.425 81.675) (end 100.3 81.675) (width 0.3) (layer "F.Cu") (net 1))
 (segment (start 87.279 75.896) (end 88.27 75.896) (width 0.3) (layer "F.Cu") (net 1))
 (segment (start 113.125 75.475) (end 112.65 75) (width 0.3) (layer "F.Cu") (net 1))
 (segment (start 91.425 81.675) (end 88.27 78.52) (width 0.3) (layer "F.Cu") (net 1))
 (segment (start 113.125 77.5) (end 113.125 75.475) (width 0.3) (layer "F.Cu") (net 1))
 (segment (start 95.6 81.675) (end 91.425 81.675) (width 0.3) (layer "F.Cu") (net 1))
 (segment (start 108.1 75) (end 101.425 81.675) (width 0.3) (layer "F.Cu") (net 1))
 (segment (start 86.25 77.9) (end 86.25 76.925) (width 0.3) (layer "F.Cu") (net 1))
 (via (at 95.6 81.675) (size 0.6) (drill 0.3) (layers "F.Cu" "B.Cu") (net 1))
 (via (at 86.25 77.9) (size 0.6) (drill 0.3) (layers "F.Cu" "B.Cu") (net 1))
 (via (at 86.225 106.225) (size 0.6) (drill 0.3) (layers "F.Cu" "B.Cu") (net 1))
 (via (at 100.3 81.675) (size 0.6) (drill 0.3) (layers "F.Cu" "B.Cu") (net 1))
 (segment (start 86.225 77.941) (end 86.225 77.925) (width 0.3) (layer "B.Cu") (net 1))
 (segment (start 86.225 106.225) (end 86.225 77.941) (width 0.3) (layer "B.Cu") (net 1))
 (segment (start 86.225 77.925) (end 86.25 77.9) (width 0.3) (layer "B.Cu") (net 1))
 (segment (start 95.6 81.675) (end 100.3 81.675) (width 0.3) (layer "B.Cu") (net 1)))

